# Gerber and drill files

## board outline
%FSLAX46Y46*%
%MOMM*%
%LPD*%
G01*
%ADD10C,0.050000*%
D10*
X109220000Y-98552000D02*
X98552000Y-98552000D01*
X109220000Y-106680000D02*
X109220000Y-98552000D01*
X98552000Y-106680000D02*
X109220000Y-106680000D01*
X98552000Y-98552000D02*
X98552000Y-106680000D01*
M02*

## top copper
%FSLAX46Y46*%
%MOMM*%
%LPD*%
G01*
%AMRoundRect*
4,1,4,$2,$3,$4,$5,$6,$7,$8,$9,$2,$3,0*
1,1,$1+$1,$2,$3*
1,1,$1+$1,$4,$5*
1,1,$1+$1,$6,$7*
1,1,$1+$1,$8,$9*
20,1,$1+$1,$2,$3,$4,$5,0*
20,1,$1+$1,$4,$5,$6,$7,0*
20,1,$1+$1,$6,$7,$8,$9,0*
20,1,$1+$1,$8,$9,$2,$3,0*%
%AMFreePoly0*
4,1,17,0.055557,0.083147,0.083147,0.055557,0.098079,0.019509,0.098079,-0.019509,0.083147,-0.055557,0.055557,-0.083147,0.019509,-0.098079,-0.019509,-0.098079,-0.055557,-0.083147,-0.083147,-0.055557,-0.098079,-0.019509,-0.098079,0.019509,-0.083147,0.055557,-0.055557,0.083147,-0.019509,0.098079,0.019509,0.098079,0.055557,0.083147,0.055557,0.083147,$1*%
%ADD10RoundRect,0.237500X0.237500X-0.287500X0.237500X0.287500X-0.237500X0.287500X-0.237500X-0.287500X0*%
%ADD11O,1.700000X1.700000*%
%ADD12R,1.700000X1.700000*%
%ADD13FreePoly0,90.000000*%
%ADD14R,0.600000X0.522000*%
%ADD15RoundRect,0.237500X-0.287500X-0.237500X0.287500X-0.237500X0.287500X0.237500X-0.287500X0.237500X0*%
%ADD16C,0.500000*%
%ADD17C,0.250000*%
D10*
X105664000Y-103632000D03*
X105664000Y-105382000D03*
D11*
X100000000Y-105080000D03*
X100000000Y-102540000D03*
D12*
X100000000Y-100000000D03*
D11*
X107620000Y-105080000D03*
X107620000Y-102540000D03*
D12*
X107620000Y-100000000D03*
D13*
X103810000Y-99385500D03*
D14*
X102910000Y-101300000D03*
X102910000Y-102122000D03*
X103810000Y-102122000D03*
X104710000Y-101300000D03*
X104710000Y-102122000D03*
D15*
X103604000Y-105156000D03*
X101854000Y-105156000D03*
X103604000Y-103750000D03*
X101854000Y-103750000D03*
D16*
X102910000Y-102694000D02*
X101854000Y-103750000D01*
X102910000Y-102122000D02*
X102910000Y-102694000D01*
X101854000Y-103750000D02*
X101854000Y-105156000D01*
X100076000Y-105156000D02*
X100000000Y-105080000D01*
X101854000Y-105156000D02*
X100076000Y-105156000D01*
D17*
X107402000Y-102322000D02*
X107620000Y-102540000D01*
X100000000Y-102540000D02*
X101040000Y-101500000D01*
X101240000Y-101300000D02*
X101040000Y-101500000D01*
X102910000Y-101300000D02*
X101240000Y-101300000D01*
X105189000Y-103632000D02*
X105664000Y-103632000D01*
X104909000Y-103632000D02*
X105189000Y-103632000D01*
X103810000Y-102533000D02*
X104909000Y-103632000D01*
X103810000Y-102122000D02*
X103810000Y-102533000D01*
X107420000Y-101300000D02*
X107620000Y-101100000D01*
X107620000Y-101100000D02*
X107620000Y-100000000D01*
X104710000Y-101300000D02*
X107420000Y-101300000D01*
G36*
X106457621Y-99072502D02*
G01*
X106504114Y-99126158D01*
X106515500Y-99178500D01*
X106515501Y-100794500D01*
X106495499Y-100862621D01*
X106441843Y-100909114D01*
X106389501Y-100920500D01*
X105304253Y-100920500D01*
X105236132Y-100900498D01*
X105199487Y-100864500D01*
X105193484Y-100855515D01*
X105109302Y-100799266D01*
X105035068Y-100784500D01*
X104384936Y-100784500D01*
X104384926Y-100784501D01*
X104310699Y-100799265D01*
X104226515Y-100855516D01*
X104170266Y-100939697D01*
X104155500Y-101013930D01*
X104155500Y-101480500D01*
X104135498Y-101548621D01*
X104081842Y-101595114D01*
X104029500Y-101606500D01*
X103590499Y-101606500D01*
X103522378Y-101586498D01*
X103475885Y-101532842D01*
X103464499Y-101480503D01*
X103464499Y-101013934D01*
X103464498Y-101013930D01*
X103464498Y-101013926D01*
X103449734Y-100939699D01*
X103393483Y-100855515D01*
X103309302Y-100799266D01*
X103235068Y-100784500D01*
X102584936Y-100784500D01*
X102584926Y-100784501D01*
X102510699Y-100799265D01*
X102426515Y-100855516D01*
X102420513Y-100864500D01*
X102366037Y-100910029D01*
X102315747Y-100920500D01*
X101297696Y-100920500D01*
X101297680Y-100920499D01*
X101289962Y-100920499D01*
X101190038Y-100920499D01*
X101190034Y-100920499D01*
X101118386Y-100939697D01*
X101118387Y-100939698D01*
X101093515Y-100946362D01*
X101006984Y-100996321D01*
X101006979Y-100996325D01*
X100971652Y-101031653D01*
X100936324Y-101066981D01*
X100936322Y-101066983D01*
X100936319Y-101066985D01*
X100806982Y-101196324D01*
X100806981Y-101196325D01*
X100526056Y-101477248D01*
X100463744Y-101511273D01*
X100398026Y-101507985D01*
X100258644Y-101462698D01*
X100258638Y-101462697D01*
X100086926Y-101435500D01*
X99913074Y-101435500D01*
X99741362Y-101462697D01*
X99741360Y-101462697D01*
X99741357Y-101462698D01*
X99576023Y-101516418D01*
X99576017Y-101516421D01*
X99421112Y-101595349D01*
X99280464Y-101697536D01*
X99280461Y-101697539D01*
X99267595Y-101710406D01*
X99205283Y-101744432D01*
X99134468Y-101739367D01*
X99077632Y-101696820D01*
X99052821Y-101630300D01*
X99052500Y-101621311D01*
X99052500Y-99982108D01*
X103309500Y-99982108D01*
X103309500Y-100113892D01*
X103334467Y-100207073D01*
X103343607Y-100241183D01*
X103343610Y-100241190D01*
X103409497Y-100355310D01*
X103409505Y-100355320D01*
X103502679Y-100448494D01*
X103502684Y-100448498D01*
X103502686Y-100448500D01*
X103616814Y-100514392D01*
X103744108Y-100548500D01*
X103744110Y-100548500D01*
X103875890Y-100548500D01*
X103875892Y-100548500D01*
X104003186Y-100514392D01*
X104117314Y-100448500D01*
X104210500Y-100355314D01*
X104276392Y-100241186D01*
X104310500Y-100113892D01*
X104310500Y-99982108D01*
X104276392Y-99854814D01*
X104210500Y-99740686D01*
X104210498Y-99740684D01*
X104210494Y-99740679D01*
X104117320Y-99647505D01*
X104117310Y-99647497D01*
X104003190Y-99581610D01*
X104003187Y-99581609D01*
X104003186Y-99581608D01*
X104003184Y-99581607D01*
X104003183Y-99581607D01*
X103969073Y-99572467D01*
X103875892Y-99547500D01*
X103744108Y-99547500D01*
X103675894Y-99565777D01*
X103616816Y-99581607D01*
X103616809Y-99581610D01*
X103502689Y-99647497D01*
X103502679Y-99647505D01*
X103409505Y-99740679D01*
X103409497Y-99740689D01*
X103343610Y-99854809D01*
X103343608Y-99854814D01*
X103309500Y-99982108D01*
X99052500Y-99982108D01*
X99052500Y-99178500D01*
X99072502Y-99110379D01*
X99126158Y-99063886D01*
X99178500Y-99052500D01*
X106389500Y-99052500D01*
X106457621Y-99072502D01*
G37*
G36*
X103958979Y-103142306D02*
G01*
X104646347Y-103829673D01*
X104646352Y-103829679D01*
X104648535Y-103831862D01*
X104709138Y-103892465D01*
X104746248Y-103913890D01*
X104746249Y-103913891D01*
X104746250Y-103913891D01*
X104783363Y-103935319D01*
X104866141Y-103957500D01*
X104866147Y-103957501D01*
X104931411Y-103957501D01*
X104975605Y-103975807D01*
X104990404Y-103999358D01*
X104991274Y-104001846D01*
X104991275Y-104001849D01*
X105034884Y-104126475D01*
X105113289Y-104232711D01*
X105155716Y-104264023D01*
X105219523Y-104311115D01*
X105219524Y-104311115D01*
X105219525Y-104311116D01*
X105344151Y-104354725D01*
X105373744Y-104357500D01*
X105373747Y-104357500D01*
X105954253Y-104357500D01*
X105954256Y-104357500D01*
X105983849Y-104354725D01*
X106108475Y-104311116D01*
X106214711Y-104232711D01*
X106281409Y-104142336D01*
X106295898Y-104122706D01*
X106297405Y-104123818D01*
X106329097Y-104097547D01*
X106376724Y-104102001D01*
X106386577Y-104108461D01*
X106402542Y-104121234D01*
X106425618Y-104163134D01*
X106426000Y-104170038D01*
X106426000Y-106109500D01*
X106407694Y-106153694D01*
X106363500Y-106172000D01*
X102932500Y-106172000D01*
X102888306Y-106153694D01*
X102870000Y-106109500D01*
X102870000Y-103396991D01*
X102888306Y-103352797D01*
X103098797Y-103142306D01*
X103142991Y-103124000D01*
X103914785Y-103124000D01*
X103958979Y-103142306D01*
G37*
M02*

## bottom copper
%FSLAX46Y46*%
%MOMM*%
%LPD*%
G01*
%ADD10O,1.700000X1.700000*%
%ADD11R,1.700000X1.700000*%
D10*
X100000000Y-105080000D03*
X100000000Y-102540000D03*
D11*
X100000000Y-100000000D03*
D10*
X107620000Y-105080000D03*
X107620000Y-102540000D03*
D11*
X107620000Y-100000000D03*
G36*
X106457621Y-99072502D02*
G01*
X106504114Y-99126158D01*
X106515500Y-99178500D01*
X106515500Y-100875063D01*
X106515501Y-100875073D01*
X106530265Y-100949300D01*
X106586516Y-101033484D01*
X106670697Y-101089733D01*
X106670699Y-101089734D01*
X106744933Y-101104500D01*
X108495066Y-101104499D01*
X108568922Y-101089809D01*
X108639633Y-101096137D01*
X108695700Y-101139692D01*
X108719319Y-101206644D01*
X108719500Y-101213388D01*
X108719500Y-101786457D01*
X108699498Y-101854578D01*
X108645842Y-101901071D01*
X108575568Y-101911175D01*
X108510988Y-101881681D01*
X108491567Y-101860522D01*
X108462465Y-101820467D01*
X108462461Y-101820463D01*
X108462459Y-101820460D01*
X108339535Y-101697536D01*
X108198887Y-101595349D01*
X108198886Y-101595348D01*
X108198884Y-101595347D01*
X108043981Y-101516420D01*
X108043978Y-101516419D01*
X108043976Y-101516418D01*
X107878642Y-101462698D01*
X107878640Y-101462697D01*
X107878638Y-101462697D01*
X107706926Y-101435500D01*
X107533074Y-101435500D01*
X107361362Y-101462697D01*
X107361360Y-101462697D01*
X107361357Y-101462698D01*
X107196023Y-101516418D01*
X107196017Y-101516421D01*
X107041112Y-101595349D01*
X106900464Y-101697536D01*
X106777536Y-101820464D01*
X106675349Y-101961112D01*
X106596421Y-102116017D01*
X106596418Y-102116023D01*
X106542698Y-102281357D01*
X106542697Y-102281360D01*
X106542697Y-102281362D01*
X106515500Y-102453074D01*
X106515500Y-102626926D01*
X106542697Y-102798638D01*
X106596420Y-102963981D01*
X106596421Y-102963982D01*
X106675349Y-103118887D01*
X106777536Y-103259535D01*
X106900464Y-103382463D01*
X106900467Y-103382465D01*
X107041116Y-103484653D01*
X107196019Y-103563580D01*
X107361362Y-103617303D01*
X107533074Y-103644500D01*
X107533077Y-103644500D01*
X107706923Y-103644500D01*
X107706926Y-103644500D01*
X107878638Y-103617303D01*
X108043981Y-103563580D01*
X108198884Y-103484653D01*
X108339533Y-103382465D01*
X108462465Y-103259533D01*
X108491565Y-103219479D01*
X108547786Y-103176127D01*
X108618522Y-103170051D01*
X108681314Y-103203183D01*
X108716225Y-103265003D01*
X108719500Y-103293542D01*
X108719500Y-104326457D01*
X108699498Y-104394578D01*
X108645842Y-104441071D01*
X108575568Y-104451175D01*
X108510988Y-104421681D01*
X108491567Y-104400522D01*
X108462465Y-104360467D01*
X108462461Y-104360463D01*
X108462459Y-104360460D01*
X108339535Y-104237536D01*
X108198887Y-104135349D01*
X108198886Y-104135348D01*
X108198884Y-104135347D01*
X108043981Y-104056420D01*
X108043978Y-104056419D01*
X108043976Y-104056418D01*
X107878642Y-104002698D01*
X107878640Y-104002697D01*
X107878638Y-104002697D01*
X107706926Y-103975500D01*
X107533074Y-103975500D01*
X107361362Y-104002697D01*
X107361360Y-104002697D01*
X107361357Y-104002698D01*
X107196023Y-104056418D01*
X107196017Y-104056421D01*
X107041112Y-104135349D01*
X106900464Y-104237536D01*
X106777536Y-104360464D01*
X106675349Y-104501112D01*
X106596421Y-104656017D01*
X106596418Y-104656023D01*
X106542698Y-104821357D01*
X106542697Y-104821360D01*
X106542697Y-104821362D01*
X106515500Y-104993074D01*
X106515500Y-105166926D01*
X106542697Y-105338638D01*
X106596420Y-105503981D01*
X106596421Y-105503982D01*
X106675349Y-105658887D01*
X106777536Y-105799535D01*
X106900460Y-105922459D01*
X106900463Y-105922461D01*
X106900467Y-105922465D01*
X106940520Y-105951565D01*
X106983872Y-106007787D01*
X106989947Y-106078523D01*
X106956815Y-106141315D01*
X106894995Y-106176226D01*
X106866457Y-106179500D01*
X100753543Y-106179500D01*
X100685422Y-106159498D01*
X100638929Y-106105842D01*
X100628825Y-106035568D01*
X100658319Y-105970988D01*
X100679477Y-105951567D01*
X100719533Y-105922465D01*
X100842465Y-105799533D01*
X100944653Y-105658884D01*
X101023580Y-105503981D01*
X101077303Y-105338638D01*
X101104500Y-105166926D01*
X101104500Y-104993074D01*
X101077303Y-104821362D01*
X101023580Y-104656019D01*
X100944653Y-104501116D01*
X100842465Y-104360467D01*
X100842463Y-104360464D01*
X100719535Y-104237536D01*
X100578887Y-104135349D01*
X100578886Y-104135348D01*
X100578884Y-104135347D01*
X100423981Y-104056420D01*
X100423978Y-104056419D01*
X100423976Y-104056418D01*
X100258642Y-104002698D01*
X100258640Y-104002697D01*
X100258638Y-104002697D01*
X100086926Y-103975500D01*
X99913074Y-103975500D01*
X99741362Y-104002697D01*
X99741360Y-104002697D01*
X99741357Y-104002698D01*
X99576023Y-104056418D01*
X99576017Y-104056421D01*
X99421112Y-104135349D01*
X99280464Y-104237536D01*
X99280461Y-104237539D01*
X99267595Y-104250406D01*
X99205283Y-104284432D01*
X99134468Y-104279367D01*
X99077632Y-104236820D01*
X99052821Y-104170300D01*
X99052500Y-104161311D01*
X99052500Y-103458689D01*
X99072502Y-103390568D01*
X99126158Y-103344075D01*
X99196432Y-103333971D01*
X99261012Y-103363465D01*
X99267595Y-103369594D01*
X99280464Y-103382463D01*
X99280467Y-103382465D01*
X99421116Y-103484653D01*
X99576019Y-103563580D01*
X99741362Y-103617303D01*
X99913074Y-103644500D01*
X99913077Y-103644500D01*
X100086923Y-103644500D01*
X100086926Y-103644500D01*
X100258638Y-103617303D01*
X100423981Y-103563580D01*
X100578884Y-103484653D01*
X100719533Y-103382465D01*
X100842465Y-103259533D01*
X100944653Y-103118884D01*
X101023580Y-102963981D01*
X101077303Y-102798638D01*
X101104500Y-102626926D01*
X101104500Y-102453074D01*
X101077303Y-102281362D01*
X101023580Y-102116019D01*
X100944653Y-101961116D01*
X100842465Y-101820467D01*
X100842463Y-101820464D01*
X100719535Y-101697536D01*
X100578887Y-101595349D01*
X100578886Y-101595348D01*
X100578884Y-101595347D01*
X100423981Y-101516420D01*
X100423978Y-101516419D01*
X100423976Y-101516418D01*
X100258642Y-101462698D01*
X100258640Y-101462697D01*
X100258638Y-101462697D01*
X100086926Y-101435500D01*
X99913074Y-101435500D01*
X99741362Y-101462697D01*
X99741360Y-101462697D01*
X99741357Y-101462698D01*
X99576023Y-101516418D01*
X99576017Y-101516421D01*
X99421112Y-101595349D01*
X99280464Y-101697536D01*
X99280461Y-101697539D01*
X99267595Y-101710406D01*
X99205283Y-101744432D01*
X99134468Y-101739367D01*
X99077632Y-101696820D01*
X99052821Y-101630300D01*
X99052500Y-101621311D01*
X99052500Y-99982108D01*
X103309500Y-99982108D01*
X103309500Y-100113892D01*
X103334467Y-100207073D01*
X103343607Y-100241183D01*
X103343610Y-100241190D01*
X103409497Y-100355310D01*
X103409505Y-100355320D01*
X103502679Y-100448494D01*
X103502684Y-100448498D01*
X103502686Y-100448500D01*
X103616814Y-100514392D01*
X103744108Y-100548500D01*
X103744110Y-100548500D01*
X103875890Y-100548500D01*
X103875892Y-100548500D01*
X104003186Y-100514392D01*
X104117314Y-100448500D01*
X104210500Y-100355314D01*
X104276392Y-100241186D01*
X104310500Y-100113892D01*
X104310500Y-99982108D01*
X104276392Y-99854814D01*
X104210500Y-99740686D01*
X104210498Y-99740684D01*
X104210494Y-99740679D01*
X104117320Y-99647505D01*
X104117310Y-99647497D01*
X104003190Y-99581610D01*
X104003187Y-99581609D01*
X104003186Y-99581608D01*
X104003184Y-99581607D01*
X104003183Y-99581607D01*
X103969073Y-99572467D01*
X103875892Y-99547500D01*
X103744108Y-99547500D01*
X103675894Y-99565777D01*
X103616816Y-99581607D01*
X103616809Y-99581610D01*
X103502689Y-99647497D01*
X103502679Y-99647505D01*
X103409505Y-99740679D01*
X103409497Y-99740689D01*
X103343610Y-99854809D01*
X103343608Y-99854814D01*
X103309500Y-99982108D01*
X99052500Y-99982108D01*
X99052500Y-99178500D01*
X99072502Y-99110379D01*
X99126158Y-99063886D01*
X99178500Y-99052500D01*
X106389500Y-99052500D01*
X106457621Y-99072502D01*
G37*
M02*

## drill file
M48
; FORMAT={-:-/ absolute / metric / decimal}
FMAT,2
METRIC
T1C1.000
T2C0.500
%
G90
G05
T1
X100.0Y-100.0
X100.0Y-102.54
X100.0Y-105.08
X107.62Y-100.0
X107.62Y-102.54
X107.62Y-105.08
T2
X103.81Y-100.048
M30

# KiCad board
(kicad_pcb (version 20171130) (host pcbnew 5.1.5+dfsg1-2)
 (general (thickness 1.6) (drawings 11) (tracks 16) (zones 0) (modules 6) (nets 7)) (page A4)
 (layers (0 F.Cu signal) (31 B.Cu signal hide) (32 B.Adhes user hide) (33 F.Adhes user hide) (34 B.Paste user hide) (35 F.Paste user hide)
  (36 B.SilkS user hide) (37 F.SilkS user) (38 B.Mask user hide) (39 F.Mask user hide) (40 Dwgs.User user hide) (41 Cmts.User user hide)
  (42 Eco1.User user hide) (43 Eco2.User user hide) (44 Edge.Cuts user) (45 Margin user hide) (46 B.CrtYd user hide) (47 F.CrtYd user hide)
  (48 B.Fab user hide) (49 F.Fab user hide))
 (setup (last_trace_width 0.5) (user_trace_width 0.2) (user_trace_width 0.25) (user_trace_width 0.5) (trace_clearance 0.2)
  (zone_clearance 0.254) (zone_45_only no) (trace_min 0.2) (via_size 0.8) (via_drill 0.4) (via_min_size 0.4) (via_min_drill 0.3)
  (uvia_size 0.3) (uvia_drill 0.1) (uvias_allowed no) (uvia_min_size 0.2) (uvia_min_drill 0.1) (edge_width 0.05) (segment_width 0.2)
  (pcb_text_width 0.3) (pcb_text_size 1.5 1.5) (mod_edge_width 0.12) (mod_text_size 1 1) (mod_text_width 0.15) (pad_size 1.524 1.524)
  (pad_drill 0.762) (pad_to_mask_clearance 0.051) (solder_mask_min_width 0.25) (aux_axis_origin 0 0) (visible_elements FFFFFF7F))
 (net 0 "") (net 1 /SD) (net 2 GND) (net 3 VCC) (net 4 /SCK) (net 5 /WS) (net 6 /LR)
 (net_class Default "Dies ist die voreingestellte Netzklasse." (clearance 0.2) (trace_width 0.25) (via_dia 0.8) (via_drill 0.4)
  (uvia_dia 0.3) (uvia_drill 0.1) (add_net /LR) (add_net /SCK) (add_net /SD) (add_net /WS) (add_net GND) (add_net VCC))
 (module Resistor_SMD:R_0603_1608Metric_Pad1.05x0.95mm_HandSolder (layer F.Cu) (at 105.664 104.507 90)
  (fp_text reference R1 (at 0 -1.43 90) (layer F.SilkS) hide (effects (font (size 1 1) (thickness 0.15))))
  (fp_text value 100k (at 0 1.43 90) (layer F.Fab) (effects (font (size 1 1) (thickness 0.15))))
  (pad 2 smd roundrect (at 0.875 0 90) (size 1.05 0.95) (layers F.Cu F.Paste F.Mask) (roundrect_rratio 0.25) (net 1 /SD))
  (pad 1 smd roundrect (at -0.875 0 90) (size 1.05 0.95) (layers F.Cu F.Paste F.Mask) (roundrect_rratio 0.25) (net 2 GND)))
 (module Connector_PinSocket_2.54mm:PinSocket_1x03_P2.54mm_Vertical (layer F.Cu) (at 100 100)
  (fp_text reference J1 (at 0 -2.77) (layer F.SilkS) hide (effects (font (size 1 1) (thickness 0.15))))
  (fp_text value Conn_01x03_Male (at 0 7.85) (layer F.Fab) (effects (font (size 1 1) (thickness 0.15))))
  (pad 3 thru_hole oval (at 0 5.08) (size 1.7 1.7) (drill 1) (layers *.Cu *.Mask) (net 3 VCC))
  (pad 2 thru_hole oval (at 0 2.54) (size 1.7 1.7) (drill 1) (layers *.Cu *.Mask) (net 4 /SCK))
  (pad 1 thru_hole rect (at 0 0) (size 1.7 1.7) (drill 1) (layers *.Cu *.Mask) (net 2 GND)))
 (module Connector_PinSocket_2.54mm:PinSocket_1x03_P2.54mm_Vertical (layer F.Cu) (at 107.62 100)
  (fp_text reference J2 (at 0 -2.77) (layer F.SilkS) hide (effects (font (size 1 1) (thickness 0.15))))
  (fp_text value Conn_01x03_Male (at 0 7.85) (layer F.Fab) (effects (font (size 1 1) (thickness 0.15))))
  (pad 3 thru_hole oval (at 0 5.08) (size 1.7 1.7) (drill 1) (layers *.Cu *.Mask) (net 1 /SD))
  (pad 2 thru_hole oval (at 0 2.54) (size 1.7 1.7) (drill 1) (layers *.Cu *.Mask) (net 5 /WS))
  (pad 1 thru_hole rect (at 0 0) (size 1.7 1.7) (drill 1) (layers *.Cu *.Mask) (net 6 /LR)))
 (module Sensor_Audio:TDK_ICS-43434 (layer F.Cu) (at 103.81 101.3 90)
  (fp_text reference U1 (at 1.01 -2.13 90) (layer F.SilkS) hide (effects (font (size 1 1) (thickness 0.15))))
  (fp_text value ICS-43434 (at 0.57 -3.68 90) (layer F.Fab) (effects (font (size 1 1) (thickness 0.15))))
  (pad 3 smd custom (at 1.9145 0 90) (size 0.2 0.2) (layers F.Cu F.Mask) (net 2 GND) (zone_connect 2)
   (options (clearance outline) (anchor circle)) (primitives))
  (pad "" np_thru_hole circle (at 1.252 0 90) (size 0.5 0.5) (drill 0.5) (layers *.Cu *.Mask) (zone_connect 0))
  (pad 4 smd rect (at 0 -0.9 90) (size 0.522 0.6) (layers F.Cu F.Paste F.Mask) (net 4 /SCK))
  (pad 5 smd rect (at -0.822 -0.9 90) (size 0.522 0.6) (layers F.Cu F.Paste F.Mask) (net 3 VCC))
  (pad 6 smd rect (at -0.822 0 90) (size 0.522 0.6) (layers F.Cu F.Paste F.Mask) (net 1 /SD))
  (pad 2 smd rect (at 0 0.9 90) (size 0.522 0.6) (layers F.Cu F.Paste F.Mask) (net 6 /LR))
  (pad 1 smd rect (at -0.822 0.9 90) (size 0.522 0.6) (layers F.Cu F.Paste F.Mask) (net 5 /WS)))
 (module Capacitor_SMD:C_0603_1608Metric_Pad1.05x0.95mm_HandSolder (layer F.Cu) (at 102.729 105.156)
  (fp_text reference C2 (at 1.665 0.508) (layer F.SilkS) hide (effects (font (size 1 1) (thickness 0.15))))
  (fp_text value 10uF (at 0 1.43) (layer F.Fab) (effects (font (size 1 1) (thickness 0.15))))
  (pad 2 smd roundrect (at 0.875 0) (size 1.05 0.95) (layers F.Cu F.Paste F.Mask) (roundrect_rratio 0.25) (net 2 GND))
  (pad 1 smd roundrect (at -0.875 0) (size 1.05 0.95) (layers F.Cu F.Paste F.Mask) (roundrect_rratio 0.25) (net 3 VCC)))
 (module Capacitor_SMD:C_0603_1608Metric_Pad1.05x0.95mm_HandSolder (layer F.Cu) (at 102.729 103.75)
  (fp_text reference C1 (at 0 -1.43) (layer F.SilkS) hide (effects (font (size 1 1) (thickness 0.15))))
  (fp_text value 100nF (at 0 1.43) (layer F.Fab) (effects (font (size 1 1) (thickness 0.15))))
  (pad 2 smd roundrect (at 0.875 0) (size 1.05 0.95) (layers F.Cu F.Paste F.Mask) (roundrect_rratio 0.25) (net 2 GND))
  (pad 1 smd roundrect (at -0.875 0) (size 1.05 0.95) (layers F.Cu F.Paste F.Mask) (roundrect_rratio 0.25) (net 3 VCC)))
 (gr_line (start 109.22 98.552) (end 98.552 98.552) (layer Edge.Cuts) (width 0.05))
 (gr_line (start 109.22 106.68) (end 109.22 98.552) (layer Edge.Cuts) (width 0.05))
 (gr_line (start 98.552 106.68) (end 109.22 106.68) (layer Edge.Cuts) (width 0.05))
 (gr_line (start 98.552 98.552) (end 98.552 106.68) (layer Edge.Cuts) (width 0.05))
 (segment (start 102.91 102.694) (end 101.854 103.75) (width 0.5) (layer F.Cu) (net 3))
 (segment (start 102.91 102.122) (end 102.91 102.694) (width 0.5) (layer F.Cu) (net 3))
 (segment (start 101.854 103.75) (end 101.854 105.156) (width 0.5) (layer F.Cu) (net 3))
 (segment (start 100.076 105.156) (end 100 105.08) (width 0.5) (layer F.Cu) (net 3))
 (segment (start 101.854 105.156) (end 100.076 105.156) (width 0.5) (layer F.Cu) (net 3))
 (segment (start 107.402 102.322) (end 107.62 102.54) (width 0.25) (layer F.Cu) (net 5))
 (segment (start 100 102.54) (end 101.04 101.5) (width 0.25) (layer F.Cu) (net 4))
 (segment (start 101.24 101.3) (end 101.04 101.5) (width 0.25) (layer F.Cu) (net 4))
 (segment (start 102.91 101.3) (end 101.24 101.3) (width 0.25) (layer F.Cu) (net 4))
 (segment (start 105.189 103.632) (end 105.664 103.632) (width 0.25) (layer F.Cu) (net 1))
 (segment (start 104.909 103.632) (end 105.189 103.632) (width 0.25) (layer F.Cu) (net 1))
 (segment (start 103.81 102.533) (end 104.909 103.632) (width 0.25) (layer F.Cu) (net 1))
 (segment (start 103.81 102.122) (end 103.81 102.533) (width 0.25) (layer F.Cu) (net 1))
 (segment (start 107.42 101.3) (end 107.62 101.1) (width 0.25) (layer F.Cu) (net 6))
 (segment (start 107.62 101.1) (end 107.62 100) (width 0.25) (layer F.Cu) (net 6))
 (segment (start 104.71 101.3) (end 107.42 101.3) (width 0.25) (layer F.Cu) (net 6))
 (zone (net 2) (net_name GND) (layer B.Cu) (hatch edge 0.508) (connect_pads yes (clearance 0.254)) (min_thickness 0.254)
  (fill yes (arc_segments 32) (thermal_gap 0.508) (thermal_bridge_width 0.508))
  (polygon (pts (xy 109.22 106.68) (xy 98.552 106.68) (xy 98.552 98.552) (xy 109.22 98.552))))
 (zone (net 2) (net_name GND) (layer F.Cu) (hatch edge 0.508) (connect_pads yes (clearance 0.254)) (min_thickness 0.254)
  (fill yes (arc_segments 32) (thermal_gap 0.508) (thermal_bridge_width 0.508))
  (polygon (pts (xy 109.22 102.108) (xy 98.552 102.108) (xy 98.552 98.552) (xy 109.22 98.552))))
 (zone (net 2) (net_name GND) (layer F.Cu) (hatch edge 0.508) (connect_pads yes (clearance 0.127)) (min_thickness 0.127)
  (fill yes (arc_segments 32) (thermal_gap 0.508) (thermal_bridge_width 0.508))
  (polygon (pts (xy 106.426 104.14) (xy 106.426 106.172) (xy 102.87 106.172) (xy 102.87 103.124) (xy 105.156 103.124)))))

